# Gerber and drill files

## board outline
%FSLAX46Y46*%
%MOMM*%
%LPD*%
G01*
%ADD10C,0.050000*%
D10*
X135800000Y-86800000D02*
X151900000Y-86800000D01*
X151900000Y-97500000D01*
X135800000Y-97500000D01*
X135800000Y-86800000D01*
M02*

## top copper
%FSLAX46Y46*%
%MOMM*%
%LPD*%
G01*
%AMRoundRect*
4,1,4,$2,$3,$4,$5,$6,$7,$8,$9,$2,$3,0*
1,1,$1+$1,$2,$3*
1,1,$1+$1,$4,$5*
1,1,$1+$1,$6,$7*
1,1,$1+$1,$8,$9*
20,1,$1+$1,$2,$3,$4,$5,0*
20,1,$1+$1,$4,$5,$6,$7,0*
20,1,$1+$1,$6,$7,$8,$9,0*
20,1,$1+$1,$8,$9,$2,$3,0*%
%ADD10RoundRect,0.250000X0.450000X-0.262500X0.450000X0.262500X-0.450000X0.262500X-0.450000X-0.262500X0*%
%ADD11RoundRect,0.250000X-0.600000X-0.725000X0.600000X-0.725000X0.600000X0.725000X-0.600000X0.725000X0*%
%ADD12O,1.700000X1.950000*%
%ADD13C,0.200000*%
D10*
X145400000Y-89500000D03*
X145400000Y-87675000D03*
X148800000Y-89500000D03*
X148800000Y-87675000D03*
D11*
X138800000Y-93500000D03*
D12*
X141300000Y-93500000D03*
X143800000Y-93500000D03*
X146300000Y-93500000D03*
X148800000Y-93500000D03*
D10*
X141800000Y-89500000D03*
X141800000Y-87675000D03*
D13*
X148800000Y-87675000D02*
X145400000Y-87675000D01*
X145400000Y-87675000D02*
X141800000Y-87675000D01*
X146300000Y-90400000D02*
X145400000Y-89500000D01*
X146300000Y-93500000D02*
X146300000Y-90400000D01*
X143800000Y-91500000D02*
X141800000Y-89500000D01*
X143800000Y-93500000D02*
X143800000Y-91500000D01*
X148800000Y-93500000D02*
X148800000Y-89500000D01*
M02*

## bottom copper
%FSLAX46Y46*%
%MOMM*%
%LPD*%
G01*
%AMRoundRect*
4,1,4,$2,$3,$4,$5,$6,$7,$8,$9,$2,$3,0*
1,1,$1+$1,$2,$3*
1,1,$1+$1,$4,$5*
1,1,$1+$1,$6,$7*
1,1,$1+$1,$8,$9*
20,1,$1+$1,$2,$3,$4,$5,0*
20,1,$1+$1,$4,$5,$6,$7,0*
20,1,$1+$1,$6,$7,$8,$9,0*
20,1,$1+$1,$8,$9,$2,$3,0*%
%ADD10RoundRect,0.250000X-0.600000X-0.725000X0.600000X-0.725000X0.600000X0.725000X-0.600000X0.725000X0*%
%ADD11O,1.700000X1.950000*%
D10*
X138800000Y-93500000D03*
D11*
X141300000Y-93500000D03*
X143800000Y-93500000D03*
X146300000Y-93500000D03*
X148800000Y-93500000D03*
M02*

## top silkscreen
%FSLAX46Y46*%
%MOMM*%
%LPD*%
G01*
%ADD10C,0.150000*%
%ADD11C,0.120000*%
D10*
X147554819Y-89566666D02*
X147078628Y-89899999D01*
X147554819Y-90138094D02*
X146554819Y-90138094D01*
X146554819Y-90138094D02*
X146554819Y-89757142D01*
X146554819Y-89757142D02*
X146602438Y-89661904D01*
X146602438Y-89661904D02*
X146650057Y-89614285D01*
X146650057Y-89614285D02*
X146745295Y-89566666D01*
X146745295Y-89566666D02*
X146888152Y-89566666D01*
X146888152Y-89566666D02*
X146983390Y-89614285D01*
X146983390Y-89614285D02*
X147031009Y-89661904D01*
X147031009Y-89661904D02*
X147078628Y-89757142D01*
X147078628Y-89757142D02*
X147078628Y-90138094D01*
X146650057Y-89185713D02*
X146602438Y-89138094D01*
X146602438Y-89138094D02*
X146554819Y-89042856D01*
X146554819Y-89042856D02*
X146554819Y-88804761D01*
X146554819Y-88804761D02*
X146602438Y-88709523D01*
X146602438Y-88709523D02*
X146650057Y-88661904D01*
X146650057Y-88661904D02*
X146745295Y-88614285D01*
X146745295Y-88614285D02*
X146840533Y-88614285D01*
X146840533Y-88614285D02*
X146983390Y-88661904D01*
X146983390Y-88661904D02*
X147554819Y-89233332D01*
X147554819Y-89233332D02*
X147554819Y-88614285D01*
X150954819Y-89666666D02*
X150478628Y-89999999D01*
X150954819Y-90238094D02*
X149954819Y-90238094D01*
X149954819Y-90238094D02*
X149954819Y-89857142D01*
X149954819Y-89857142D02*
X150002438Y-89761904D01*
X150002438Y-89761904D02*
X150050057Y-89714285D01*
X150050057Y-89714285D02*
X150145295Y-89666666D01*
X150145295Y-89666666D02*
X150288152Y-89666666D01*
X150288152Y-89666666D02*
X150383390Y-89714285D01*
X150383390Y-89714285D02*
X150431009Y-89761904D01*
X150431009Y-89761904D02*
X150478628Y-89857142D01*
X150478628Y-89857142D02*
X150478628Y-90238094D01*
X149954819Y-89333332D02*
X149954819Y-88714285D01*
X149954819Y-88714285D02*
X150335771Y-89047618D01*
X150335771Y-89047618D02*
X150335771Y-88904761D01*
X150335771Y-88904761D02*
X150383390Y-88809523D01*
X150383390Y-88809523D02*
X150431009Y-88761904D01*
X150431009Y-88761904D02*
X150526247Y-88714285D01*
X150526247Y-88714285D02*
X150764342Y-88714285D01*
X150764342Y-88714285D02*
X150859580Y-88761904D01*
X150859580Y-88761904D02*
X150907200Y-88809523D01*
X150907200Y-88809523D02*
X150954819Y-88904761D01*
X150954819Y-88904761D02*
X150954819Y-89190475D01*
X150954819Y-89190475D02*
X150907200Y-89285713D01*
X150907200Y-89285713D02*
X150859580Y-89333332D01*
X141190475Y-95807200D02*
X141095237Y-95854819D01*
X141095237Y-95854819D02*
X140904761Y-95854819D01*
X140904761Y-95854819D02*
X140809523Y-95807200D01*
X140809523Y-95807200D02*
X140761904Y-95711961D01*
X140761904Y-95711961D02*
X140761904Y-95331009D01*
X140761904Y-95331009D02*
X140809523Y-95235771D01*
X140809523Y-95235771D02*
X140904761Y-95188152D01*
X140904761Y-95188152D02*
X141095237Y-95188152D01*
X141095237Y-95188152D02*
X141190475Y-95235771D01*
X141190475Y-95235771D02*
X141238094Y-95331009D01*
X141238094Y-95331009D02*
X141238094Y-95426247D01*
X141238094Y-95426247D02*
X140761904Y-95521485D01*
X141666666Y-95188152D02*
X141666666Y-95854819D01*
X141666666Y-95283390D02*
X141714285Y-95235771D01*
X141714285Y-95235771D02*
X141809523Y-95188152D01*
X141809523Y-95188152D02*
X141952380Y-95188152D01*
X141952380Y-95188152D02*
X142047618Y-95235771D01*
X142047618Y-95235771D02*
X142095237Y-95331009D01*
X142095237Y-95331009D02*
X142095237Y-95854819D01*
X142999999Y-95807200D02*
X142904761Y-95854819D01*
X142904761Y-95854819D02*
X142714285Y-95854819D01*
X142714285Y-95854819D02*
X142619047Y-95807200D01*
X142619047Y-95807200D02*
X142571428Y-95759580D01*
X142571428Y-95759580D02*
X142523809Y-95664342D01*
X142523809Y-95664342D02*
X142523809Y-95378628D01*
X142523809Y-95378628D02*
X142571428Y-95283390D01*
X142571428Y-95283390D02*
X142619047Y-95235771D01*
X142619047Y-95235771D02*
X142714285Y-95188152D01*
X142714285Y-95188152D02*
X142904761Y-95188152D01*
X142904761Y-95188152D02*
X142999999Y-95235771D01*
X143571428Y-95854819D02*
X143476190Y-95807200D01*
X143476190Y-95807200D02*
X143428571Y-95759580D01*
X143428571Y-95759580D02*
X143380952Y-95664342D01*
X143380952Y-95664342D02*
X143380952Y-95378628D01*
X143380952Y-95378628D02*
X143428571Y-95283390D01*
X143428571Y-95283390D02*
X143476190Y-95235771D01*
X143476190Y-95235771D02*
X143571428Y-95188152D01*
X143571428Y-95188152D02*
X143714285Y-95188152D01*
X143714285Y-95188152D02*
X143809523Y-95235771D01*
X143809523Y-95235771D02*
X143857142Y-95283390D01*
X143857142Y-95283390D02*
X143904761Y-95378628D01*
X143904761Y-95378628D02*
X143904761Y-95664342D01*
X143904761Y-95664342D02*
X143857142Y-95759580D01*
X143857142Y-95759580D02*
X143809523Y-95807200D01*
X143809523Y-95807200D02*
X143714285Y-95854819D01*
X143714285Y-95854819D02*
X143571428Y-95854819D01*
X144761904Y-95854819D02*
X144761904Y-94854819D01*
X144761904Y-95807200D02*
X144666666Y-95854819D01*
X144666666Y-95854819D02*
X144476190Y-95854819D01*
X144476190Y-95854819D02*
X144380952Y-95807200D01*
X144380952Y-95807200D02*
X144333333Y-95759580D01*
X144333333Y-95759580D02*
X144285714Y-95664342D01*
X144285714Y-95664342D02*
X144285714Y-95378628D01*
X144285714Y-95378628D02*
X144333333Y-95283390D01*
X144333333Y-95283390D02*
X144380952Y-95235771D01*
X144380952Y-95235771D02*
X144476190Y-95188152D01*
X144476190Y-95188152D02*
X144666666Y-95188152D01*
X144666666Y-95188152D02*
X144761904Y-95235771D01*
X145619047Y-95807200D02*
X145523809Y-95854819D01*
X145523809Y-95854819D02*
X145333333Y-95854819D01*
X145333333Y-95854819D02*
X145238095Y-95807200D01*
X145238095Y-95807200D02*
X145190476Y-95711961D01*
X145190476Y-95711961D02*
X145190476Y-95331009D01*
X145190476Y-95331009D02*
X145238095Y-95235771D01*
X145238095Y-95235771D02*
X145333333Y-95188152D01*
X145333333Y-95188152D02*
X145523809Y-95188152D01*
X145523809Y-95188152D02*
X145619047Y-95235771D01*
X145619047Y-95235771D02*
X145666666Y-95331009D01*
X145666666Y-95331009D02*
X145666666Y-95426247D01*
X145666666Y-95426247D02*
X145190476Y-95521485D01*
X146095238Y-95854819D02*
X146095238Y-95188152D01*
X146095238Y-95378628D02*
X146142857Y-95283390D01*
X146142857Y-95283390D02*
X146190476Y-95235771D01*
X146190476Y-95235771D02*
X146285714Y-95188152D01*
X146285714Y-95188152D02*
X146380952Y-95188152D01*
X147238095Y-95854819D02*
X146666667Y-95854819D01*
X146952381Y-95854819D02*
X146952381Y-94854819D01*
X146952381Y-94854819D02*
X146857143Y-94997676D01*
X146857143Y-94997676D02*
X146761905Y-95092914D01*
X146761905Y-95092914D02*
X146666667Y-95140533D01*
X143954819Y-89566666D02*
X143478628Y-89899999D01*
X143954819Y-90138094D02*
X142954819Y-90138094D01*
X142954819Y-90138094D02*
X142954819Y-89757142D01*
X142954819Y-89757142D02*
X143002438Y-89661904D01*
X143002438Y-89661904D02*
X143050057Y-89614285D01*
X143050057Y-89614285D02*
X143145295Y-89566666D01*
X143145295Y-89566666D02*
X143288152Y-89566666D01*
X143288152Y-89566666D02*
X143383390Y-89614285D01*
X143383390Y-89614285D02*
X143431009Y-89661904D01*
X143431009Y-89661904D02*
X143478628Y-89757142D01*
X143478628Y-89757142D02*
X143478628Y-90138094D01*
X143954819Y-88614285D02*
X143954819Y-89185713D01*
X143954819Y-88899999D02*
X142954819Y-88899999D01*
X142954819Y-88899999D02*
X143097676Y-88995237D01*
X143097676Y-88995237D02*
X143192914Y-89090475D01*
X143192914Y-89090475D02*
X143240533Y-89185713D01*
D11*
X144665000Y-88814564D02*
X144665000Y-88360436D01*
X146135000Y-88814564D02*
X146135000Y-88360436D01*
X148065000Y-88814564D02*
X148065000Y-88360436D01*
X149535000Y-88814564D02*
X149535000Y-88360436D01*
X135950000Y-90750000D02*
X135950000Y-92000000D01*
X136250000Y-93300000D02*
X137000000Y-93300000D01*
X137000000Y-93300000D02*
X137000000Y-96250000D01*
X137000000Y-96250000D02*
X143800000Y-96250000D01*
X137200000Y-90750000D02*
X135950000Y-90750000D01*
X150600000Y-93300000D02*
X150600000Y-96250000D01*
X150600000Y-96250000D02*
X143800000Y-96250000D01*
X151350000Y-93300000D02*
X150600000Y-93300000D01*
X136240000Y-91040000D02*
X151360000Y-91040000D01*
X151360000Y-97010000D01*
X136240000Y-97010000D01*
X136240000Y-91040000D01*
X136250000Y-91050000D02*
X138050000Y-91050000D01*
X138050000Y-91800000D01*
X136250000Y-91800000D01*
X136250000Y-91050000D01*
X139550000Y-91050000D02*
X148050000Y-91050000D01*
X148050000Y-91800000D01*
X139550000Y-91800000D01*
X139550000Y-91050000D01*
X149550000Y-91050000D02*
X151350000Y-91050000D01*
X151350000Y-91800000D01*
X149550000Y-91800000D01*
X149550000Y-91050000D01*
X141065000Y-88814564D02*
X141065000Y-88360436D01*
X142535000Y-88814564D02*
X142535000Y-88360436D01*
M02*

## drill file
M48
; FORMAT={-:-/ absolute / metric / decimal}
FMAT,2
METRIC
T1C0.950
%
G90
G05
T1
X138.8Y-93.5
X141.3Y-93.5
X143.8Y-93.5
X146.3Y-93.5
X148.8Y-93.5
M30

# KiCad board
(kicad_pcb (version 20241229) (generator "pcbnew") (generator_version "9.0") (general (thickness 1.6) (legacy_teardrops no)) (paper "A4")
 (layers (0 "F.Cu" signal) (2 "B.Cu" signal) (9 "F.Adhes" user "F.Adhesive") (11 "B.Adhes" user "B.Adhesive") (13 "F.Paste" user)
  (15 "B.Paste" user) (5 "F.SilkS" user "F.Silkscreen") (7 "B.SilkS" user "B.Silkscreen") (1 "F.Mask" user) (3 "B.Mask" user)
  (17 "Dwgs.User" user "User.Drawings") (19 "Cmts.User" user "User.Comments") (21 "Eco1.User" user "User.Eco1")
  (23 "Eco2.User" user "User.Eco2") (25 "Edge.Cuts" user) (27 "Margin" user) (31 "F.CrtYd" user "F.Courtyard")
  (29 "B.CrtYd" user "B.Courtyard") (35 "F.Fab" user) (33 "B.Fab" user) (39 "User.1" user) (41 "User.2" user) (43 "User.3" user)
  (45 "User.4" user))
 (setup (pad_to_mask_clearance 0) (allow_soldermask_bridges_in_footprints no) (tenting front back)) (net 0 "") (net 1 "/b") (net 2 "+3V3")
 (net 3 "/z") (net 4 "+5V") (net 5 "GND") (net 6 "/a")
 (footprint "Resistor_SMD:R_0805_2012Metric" (layer "F.Cu") (at 145.4 88.5875 90)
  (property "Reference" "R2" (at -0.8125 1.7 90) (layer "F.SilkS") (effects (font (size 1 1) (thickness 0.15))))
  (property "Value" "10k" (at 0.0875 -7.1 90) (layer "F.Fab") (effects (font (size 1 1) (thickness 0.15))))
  (fp_line (start -0.227064 -0.735) (end 0.227064 -0.735) (stroke (width 0.12) (type solid)) (layer "F.SilkS"))
  (fp_line (start -0.227064 0.735) (end 0.227064 0.735) (stroke (width 0.12) (type solid)) (layer "F.SilkS"))
  (pad "1" smd roundrect (at -0.9125 0 90) (size 1.025 1.4) (layers "F.Cu" "F.Mask" "F.Paste") (roundrect_rratio 0.243902) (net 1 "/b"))
  (pad "2" smd roundrect (at 0.9125 0 90) (size 1.025 1.4) (layers "F.Cu" "F.Mask" "F.Paste") (roundrect_rratio 0.243902) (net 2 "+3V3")))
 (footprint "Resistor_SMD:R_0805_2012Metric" (layer "F.Cu") (at 148.8 88.5875 90)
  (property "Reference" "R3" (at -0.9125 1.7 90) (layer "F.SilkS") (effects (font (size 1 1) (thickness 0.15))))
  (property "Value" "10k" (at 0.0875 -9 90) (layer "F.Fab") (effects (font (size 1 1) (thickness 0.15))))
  (fp_line (start -0.227064 -0.735) (end 0.227064 -0.735) (stroke (width 0.12) (type solid)) (layer "F.SilkS"))
  (fp_line (start -0.227064 0.735) (end 0.227064 0.735) (stroke (width 0.12) (type solid)) (layer "F.SilkS"))
  (pad "1" smd roundrect (at -0.9125 0 90) (size 1.025 1.4) (layers "F.Cu" "F.Mask" "F.Paste") (roundrect_rratio 0.243902) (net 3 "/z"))
  (pad "2" smd roundrect (at 0.9125 0 90) (size 1.025 1.4) (layers "F.Cu" "F.Mask" "F.Paste") (roundrect_rratio 0.243902) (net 2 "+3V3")))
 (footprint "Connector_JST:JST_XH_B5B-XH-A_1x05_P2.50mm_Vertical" (layer "F.Cu") (at 138.8 93.5)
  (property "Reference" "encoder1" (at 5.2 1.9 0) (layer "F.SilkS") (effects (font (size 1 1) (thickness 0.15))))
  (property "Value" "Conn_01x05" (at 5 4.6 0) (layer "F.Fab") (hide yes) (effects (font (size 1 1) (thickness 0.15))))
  (fp_line (start -2.85 -2.75) (end -2.85 -1.5) (stroke (width 0.12) (type solid)) (layer "F.SilkS"))
  (fp_line (start -2.55 -0.2) (end -1.8 -0.2) (stroke (width 0.12) (type solid)) (layer "F.SilkS"))
  (fp_line (start -1.8 -0.2) (end -1.8 2.75) (stroke (width 0.12) (type solid)) (layer "F.SilkS"))
  (fp_line (start -1.8 2.75) (end 5 2.75) (stroke (width 0.12) (type solid)) (layer "F.SilkS"))
  (fp_line (start -1.6 -2.75) (end -2.85 -2.75) (stroke (width 0.12) (type solid)) (layer "F.SilkS"))
  (fp_line (start 11.8 -0.2) (end 11.8 2.75) (stroke (width 0.12) (type solid)) (layer "F.SilkS"))
  (fp_line (start 11.8 2.75) (end 5 2.75) (stroke (width 0.12) (type solid)) (layer "F.SilkS"))
  (fp_line (start 12.55 -0.2) (end 11.8 -0.2) (stroke (width 0.12) (type solid)) (layer "F.SilkS"))
  (fp_rect (start -2.56 -2.46) (end 12.56 3.51) (stroke (width 0.12) (type solid)) (fill no) (layer "F.SilkS"))
  (fp_rect (start -2.55 -2.45) (end -0.75 -1.7) (stroke (width 0.12) (type solid)) (fill no) (layer "F.SilkS"))
  (fp_rect (start 0.75 -2.45) (end 9.25 -1.7) (stroke (width 0.12) (type solid)) (fill no) (layer "F.SilkS"))
  (fp_rect (start 10.75 -2.45) (end 12.55 -1.7) (stroke (width 0.12) (type solid)) (fill no) (layer "F.SilkS"))
  (pad "1" thru_hole roundrect (at 0 0) (size 1.7 1.95) (drill 0.95) (layers "*.Cu" "*.Mask") (remove_unused_layers no)
   (roundrect_rratio 0.147059) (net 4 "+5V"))
  (pad "2" thru_hole oval (at 2.5 0) (size 1.7 1.95) (drill 0.95) (layers "*.Cu" "*.Mask") (remove_unused_layers no) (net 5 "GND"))
  (pad "3" thru_hole oval (at 5 0) (size 1.7 1.95) (drill 0.95) (layers "*.Cu" "*.Mask") (remove_unused_layers no) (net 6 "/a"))
  (pad "4" thru_hole oval (at 7.5 0) (size 1.7 1.95) (drill 0.95) (layers "*.Cu" "*.Mask") (remove_unused_layers no) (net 1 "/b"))
  (pad "5" thru_hole oval (at 10 0) (size 1.7 1.95) (drill 0.95) (layers "*.Cu" "*.Mask") (remove_unused_layers no) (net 3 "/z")))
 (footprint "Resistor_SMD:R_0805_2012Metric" (layer "F.Cu") (at 141.8 88.5875 90)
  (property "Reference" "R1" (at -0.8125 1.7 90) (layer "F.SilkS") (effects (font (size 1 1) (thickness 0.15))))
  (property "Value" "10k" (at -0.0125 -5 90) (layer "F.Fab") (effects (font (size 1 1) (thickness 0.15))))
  (fp_line (start -0.227064 -0.735) (end 0.227064 -0.735) (stroke (width 0.12) (type solid)) (layer "F.SilkS"))
  (fp_line (start -0.227064 0.735) (end 0.227064 0.735) (stroke (width 0.12) (type solid)) (layer "F.SilkS"))
  (pad "1" smd roundrect (at -0.9125 0 90) (size 1.025 1.4) (layers "F.Cu" "F.Mask" "F.Paste") (roundrect_rratio 0.243902) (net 6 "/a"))
  (pad "2" smd roundrect (at 0.9125 0 90) (size 1.025 1.4) (layers "F.Cu" "F.Mask" "F.Paste") (roundrect_rratio 0.243902) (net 2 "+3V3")))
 (gr_rect (start 135.8 86.8) (end 151.9 97.5) (stroke (width 0.05) (type default)) (fill no) (layer "Edge.Cuts"))
 (segment (start 148.8 87.675) (end 145.4 87.675) (width 0.2) (layer "F.Cu") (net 2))
 (segment (start 145.4 87.675) (end 141.8 87.675) (width 0.2) (layer "F.Cu") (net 2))
 (segment (start 146.3 90.4) (end 145.4 89.5) (width 0.2) (layer "F.Cu") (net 1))
 (segment (start 146.3 93.5) (end 146.3 90.4) (width 0.2) (layer "F.Cu") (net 1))
 (segment (start 143.8 91.5) (end 141.8 89.5) (width 0.2) (layer "F.Cu") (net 6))
 (segment (start 143.8 93.5) (end 143.8 91.5) (width 0.2) (layer "F.Cu") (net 6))
 (segment (start 148.8 93.5) (end 148.8 89.5) (width 0.2) (layer "F.Cu") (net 3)))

